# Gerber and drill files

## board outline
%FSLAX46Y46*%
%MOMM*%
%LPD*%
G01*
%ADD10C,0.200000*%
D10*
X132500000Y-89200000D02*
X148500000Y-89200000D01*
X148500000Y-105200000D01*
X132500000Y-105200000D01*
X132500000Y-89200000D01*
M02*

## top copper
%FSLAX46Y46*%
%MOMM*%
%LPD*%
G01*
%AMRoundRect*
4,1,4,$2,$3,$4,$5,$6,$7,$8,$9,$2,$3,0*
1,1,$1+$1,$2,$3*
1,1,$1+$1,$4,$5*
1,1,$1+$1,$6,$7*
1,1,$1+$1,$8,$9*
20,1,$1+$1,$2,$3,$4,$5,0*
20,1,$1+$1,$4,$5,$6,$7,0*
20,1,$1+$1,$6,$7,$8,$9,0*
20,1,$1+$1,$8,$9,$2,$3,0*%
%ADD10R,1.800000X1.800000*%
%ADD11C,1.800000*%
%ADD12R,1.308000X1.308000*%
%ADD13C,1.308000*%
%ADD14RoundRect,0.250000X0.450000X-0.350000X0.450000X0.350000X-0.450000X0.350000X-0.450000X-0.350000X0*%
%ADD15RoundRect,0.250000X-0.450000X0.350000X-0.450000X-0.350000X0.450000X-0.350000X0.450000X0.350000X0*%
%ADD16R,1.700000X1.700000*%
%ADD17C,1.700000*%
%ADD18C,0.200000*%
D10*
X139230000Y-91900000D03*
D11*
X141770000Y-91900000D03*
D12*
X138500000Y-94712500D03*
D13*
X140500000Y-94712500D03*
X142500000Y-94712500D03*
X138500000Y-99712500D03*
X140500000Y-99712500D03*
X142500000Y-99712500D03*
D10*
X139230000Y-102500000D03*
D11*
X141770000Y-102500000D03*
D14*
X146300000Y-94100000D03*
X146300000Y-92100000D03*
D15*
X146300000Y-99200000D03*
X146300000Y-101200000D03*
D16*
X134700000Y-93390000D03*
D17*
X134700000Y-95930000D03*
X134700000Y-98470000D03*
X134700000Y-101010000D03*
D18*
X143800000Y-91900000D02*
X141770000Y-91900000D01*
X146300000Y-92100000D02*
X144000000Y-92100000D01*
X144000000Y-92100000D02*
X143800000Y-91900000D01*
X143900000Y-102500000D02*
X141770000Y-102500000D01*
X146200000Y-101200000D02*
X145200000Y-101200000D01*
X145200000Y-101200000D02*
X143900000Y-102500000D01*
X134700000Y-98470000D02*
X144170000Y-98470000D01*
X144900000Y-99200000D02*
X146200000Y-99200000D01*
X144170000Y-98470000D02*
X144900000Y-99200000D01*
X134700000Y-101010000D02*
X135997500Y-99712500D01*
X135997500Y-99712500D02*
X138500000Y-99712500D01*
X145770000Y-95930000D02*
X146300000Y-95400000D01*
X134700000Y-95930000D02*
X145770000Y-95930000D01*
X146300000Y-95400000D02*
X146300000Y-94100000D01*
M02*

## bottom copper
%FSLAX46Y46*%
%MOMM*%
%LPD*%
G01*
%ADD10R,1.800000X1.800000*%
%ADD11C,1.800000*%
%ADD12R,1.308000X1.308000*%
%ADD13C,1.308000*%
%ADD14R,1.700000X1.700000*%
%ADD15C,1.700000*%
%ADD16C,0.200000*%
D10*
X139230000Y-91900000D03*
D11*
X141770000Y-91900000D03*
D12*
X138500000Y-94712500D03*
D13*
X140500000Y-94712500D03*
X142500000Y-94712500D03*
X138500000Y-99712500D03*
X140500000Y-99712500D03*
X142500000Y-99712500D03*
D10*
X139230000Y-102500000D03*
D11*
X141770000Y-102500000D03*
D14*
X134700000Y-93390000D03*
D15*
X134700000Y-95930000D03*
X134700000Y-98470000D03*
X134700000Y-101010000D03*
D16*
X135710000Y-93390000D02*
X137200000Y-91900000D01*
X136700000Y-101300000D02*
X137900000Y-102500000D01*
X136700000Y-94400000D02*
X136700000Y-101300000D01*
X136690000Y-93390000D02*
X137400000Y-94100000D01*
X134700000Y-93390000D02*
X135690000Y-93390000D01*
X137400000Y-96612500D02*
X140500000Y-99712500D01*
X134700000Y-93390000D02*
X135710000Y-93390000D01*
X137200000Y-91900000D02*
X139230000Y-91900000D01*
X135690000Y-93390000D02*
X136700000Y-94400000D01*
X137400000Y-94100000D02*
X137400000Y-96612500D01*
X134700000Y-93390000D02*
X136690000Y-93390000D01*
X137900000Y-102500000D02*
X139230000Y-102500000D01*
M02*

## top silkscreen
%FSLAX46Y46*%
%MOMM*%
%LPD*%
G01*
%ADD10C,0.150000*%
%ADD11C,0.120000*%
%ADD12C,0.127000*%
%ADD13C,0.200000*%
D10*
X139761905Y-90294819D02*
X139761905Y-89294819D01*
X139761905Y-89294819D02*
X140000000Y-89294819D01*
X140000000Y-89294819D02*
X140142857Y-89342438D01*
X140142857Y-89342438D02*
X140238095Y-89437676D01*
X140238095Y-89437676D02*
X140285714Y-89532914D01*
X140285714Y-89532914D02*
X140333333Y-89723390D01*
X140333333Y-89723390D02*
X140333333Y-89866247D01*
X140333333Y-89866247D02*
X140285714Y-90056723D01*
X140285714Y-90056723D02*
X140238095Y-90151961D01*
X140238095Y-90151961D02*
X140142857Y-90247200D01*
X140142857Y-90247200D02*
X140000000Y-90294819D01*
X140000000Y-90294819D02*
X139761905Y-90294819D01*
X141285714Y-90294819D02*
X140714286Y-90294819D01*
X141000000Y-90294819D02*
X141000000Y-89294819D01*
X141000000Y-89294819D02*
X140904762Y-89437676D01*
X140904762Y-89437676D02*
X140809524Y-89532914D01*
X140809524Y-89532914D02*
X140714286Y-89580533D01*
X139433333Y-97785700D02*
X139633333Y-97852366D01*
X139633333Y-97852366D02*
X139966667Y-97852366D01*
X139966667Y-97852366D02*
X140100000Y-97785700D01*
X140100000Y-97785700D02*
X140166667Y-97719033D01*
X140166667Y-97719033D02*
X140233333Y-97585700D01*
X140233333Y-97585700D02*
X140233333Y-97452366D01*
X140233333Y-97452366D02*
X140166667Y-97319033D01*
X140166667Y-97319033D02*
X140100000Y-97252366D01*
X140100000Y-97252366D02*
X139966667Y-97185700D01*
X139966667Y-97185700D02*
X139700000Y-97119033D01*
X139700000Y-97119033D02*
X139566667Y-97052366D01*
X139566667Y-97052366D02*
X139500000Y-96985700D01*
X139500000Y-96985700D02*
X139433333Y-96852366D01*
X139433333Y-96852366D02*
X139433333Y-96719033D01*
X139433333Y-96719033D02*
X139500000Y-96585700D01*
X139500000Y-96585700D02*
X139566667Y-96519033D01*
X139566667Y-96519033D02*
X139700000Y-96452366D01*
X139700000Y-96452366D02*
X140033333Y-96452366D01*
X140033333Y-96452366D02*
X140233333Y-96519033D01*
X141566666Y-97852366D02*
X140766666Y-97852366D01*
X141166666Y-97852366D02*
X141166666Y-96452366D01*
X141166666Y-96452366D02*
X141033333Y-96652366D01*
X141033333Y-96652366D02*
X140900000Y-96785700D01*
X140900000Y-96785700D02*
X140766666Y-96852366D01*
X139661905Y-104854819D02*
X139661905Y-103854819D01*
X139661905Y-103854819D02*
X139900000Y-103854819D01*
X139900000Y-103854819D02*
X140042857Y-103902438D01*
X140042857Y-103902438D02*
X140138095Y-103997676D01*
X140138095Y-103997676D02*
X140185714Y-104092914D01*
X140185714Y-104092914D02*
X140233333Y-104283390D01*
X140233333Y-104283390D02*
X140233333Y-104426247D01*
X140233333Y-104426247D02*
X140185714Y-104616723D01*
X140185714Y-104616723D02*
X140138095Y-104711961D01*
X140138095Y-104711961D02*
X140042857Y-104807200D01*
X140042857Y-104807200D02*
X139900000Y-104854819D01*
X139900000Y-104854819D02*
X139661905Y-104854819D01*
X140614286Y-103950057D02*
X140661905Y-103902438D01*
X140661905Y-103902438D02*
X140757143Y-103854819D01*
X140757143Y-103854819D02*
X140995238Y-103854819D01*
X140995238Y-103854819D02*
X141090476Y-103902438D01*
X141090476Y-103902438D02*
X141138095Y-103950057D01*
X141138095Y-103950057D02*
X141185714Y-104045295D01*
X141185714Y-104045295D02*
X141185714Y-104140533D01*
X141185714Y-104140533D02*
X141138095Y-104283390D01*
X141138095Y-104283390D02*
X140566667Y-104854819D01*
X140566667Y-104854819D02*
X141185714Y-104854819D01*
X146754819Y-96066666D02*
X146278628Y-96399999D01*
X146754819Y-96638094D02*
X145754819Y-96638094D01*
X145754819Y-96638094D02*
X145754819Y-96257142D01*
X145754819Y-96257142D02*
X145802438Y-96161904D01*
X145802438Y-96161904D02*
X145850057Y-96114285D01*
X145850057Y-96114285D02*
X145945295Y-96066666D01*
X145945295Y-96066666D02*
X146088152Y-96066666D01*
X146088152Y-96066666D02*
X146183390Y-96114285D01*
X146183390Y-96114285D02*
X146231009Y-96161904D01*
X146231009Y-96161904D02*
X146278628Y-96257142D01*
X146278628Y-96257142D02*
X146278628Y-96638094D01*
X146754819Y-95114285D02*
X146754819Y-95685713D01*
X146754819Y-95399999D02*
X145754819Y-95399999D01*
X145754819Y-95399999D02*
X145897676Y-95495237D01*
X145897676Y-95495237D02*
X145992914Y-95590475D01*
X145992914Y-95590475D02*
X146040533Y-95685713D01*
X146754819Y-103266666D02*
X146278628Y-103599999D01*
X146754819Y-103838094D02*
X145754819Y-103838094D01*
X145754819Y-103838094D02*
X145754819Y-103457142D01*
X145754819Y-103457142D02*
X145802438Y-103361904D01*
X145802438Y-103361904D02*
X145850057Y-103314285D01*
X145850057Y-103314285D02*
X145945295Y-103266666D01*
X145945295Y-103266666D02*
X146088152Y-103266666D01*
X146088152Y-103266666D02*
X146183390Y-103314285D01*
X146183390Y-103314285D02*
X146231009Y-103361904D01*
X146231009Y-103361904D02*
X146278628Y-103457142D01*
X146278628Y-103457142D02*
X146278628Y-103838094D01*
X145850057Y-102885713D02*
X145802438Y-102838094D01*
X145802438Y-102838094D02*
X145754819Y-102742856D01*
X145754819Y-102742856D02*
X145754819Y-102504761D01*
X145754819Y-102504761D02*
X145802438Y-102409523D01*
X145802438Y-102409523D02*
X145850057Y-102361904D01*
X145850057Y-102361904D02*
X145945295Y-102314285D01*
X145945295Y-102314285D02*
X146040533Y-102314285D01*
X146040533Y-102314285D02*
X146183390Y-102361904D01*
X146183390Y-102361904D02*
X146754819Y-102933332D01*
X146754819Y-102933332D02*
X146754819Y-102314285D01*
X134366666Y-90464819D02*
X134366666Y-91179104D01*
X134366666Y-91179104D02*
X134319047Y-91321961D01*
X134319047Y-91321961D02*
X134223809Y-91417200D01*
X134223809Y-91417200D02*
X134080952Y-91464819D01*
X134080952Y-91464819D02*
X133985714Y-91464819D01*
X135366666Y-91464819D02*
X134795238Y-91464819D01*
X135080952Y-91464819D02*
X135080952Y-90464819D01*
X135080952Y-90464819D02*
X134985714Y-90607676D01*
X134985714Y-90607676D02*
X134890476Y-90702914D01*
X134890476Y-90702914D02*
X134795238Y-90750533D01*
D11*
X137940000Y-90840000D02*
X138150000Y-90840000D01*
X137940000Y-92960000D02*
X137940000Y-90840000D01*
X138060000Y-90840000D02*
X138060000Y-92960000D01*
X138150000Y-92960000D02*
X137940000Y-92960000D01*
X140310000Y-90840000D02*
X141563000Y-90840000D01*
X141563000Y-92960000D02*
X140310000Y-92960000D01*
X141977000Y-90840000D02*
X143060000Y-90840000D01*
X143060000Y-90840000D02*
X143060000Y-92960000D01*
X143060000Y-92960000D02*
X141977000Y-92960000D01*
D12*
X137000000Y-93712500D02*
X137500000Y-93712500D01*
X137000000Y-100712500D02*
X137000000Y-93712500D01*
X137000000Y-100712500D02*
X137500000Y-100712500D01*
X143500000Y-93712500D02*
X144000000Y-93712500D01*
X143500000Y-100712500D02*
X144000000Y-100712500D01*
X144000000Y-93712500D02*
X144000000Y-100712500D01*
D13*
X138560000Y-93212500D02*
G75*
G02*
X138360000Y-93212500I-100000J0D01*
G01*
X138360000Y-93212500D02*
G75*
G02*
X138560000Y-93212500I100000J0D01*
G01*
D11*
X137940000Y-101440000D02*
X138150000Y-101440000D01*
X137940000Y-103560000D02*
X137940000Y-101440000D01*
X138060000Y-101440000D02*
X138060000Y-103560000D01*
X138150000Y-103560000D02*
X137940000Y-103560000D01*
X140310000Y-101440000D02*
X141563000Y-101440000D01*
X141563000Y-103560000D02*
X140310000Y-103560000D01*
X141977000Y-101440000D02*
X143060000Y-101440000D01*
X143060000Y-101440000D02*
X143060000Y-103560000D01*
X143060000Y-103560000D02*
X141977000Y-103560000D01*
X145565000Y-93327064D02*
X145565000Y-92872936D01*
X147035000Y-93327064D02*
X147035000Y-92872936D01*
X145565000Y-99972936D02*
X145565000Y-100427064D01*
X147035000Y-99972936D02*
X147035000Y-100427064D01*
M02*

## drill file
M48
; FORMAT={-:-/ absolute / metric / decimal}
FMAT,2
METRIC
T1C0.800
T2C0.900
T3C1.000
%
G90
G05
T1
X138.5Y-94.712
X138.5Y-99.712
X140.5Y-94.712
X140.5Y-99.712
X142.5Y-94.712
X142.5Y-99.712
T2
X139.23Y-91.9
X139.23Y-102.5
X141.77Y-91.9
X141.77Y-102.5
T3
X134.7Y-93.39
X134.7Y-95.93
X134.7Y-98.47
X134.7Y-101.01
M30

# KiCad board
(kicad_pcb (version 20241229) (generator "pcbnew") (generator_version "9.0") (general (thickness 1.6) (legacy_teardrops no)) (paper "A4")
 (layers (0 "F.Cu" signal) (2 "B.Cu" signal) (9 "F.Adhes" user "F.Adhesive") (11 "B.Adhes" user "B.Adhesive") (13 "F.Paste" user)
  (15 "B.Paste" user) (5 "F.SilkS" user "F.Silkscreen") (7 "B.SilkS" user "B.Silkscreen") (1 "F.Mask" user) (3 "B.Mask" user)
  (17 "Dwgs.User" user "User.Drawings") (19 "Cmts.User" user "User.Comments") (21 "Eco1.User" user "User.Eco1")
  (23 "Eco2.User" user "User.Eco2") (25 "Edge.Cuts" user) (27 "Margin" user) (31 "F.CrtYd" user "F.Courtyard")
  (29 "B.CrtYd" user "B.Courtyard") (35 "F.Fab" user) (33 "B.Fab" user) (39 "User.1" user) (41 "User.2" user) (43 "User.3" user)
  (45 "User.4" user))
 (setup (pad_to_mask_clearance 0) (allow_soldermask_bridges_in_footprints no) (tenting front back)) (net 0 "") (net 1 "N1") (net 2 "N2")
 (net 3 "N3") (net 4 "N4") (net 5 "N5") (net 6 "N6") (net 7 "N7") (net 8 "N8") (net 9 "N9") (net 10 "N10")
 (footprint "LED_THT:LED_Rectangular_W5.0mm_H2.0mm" (layer "F.Cu") (at 139.23 91.9)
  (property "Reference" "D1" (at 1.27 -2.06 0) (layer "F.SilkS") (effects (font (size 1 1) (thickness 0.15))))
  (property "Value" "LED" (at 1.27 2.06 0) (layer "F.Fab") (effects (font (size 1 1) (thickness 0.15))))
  (fp_line (start -1.29 -1.06) (end -1.08 -1.06) (stroke (width 0.12) (type solid)) (layer "F.SilkS"))
  (fp_line (start -1.29 1.06) (end -1.29 -1.06) (stroke (width 0.12) (type solid)) (layer "F.SilkS"))
  (fp_line (start -1.17 -1.06) (end -1.17 1.06) (stroke (width 0.12) (type solid)) (layer "F.SilkS"))
  (fp_line (start -1.08 1.06) (end -1.29 1.06) (stroke (width 0.12) (type solid)) (layer "F.SilkS"))
  (fp_line (start 1.08 -1.06) (end 2.333 -1.06) (stroke (width 0.12) (type solid)) (layer "F.SilkS"))
  (fp_line (start 2.333 1.06) (end 1.08 1.06) (stroke (width 0.12) (type solid)) (layer "F.SilkS"))
  (fp_line (start 2.747 -1.06) (end 3.83 -1.06) (stroke (width 0.12) (type solid)) (layer "F.SilkS"))
  (fp_line (start 3.83 -1.06) (end 3.83 1.06) (stroke (width 0.12) (type solid)) (layer "F.SilkS"))
  (fp_line (start 3.83 1.06) (end 2.747 1.06) (stroke (width 0.12) (type solid)) (layer "F.SilkS"))
  (pad "1" thru_hole rect (at 0 0) (size 1.8 1.8) (drill 0.9) (layers "*.Cu" "*.Mask") (remove_unused_layers no) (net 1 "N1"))
  (pad "2" thru_hole circle (at 2.54 0) (size 1.8 1.8) (drill 0.9) (layers "*.Cu" "*.Mask") (remove_unused_layers no) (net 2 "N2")))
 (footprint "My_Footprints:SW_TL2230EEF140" (layer "F.Cu") (at 140.5 97.2125)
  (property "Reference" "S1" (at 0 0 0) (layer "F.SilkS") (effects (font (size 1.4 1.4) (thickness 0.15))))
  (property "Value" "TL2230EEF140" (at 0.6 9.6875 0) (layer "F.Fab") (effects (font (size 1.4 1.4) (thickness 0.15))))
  (fp_line (start -3.5 -3.5) (end -3 -3.5) (stroke (width 0.127) (type solid)) (layer "F.SilkS"))
  (fp_line (start -3.5 3.5) (end -3.5 -3.5) (stroke (width 0.127) (type solid)) (layer "F.SilkS"))
  (fp_line (start -3.5 3.5) (end -3 3.5) (stroke (width 0.127) (type solid)) (layer "F.SilkS"))
  (fp_line (start 3 -3.5) (end 3.5 -3.5) (stroke (width 0.127) (type solid)) (layer "F.SilkS"))
  (fp_line (start 3 3.5) (end 3.5 3.5) (stroke (width 0.127) (type solid)) (layer "F.SilkS"))
  (fp_line (start 3.5 -3.5) (end 3.5 3.5) (stroke (width 0.127) (type solid)) (layer "F.SilkS"))
  (fp_circle (center -2.04 -4) (end -1.94 -4) (stroke (width 0.2) (type solid)) (fill no) (layer "F.SilkS"))
  (pad "1" thru_hole rect (at -2 -2.5) (size 1.308 1.308) (drill 0.8) (layers "*.Cu" "*.Mask") (remove_unused_layers no) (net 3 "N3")
   (solder_mask_margin 0.102))
  (pad "2" thru_hole circle (at 0 -2.5) (size 1.308 1.308) (drill 0.8) (layers "*.Cu" "*.Mask") (remove_unused_layers no) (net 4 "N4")
   (solder_mask_margin 0.102))
  (pad "3" thru_hole circle (at 2 -2.5) (size 1.308 1.308) (drill 0.8) (layers "*.Cu" "*.Mask") (remove_unused_layers no) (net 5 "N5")
   (solder_mask_margin 0.102))
  (pad "4" thru_hole circle (at -2 2.5) (size 1.308 1.308) (drill 0.8) (layers "*.Cu" "*.Mask") (remove_unused_layers no) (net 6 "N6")
   (solder_mask_margin 0.102))
  (pad "5" thru_hole circle (at 0 2.5) (size 1.308 1.308) (drill 0.8) (layers "*.Cu" "*.Mask") (remove_unused_layers no) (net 1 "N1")
   (solder_mask_margin 0.102))
  (pad "6" thru_hole circle (at 2 2.5) (size 1.308 1.308) (drill 0.8) (layers "*.Cu" "*.Mask") (remove_unused_layers no) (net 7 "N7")
   (solder_mask_margin 0.102)))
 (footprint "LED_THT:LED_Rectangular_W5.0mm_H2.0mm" (layer "F.Cu") (at 139.23 102.5)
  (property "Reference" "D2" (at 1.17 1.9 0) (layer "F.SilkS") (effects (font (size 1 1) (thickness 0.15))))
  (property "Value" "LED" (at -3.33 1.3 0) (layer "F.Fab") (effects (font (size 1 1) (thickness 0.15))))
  (fp_line (start -1.29 -1.06) (end -1.08 -1.06) (stroke (width 0.12) (type solid)) (layer "F.SilkS"))
  (fp_line (start -1.29 1.06) (end -1.29 -1.06) (stroke (width 0.12) (type solid)) (layer "F.SilkS"))
  (fp_line (start -1.17 -1.06) (end -1.17 1.06) (stroke (width 0.12) (type solid)) (layer "F.SilkS"))
  (fp_line (start -1.08 1.06) (end -1.29 1.06) (stroke (width 0.12) (type solid)) (layer "F.SilkS"))
  (fp_line (start 1.08 -1.06) (end 2.333 -1.06) (stroke (width 0.12) (type solid)) (layer "F.SilkS"))
  (fp_line (start 2.333 1.06) (end 1.08 1.06) (stroke (width 0.12) (type solid)) (layer "F.SilkS"))
  (fp_line (start 2.747 -1.06) (end 3.83 -1.06) (stroke (width 0.12) (type solid)) (layer "F.SilkS"))
  (fp_line (start 3.83 -1.06) (end 3.83 1.06) (stroke (width 0.12) (type solid)) (layer "F.SilkS"))
  (fp_line (start 3.83 1.06) (end 2.747 1.06) (stroke (width 0.12) (type solid)) (layer "F.SilkS"))
  (pad "1" thru_hole rect (at 0 0) (size 1.8 1.8) (drill 0.9) (layers "*.Cu" "*.Mask") (remove_unused_layers no) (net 1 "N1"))
  (pad "2" thru_hole circle (at 2.54 0) (size 1.8 1.8) (drill 0.9) (layers "*.Cu" "*.Mask") (remove_unused_layers no) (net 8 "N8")))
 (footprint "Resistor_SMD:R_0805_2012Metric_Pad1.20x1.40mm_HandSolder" (layer "F.Cu") (at 146.3 93.1 90)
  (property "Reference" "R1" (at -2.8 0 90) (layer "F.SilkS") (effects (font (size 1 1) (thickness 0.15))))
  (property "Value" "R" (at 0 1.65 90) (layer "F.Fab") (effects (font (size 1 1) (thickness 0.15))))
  (fp_line (start -0.227064 -0.735) (end 0.227064 -0.735) (stroke (width 0.12) (type solid)) (layer "F.SilkS"))
  (fp_line (start -0.227064 0.735) (end 0.227064 0.735) (stroke (width 0.12) (type solid)) (layer "F.SilkS"))
  (pad "1" smd roundrect (at -1 0 90) (size 1.2 1.4) (layers "F.Cu" "F.Mask" "F.Paste") (roundrect_rratio 0.208333) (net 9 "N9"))
  (pad "2" smd roundrect (at 1 0 90) (size 1.2 1.4) (layers "F.Cu" "F.Mask" "F.Paste") (roundrect_rratio 0.208333) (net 2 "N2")))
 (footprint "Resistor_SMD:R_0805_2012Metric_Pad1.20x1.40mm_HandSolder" (layer "F.Cu") (at 146.3 100.2 -90)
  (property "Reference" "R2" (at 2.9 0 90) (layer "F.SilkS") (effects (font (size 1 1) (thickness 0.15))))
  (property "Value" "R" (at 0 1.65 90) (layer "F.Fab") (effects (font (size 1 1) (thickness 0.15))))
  (fp_line (start -0.227064 0.735) (end 0.227064 0.735) (stroke (width 0.12) (type solid)) (layer "F.SilkS"))
  (fp_line (start -0.227064 -0.735) (end 0.227064 -0.735) (stroke (width 0.12) (type solid)) (layer "F.SilkS"))
  (pad "1" smd roundrect (at -1 0 270) (size 1.2 1.4) (layers "F.Cu" "F.Mask" "F.Paste") (roundrect_rratio 0.208333) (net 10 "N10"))
  (pad "2" smd roundrect (at 1 0 270) (size 1.2 1.4) (layers "F.Cu" "F.Mask" "F.Paste") (roundrect_rratio 0.208333) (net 8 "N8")))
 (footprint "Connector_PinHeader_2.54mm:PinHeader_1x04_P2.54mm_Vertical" (layer "B.Cu") (at 134.7 93.39 180)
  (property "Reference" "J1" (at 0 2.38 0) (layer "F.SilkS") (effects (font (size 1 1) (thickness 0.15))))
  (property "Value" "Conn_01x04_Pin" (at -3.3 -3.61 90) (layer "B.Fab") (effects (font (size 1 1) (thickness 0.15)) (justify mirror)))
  (pad "1" thru_hole rect (at 0 0 180) (size 1.7 1.7) (drill 1) (layers "*.Cu" "*.Mask") (remove_unused_layers no) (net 1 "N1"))
  (pad "2" thru_hole circle (at 0 -2.54 180) (size 1.7 1.7) (drill 1) (layers "*.Cu" "*.Mask") (remove_unused_layers no) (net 9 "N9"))
  (pad "3" thru_hole circle (at 0 -5.08 180) (size 1.7 1.7) (drill 1) (layers "*.Cu" "*.Mask") (remove_unused_layers no) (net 10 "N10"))
  (pad "4" thru_hole circle (at 0 -7.62 180) (size 1.7 1.7) (drill 1) (layers "*.Cu" "*.Mask") (remove_unused_layers no) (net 6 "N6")))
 (gr_rect (start 132.5 89.2) (end 148.5 105.2) (stroke (width 0.2) (type solid)) (fill no) (layer "Edge.Cuts"))
 (segment (start 135.71 93.39) (end 137.2 91.9) (width 0.2) (layer "B.Cu") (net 1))
 (segment (start 136.7 101.3) (end 137.9 102.5) (width 0.2) (layer "B.Cu") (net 1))
 (segment (start 136.7 94.4) (end 136.7 101.3) (width 0.2) (layer "B.Cu") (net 1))
 (segment (start 136.69 93.39) (end 137.4 94.1) (width 0.2) (layer "B.Cu") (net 1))
 (segment (start 134.7 93.39) (end 135.69 93.39) (width 0.2) (layer "B.Cu") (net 1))
 (segment (start 137.4 96.6125) (end 140.5 99.7125) (width 0.2) (layer "B.Cu") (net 1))
 (segment (start 134.7 93.39) (end 135.71 93.39) (width 0.2) (layer "B.Cu") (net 1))
 (segment (start 137.2 91.9) (end 139.23 91.9) (width 0.2) (layer "B.Cu") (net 1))
 (segment (start 135.69 93.39) (end 136.7 94.4) (width 0.2) (layer "B.Cu") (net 1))
 (segment (start 137.4 94.1) (end 137.4 96.6125) (width 0.2) (layer "B.Cu") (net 1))
 (segment (start 134.7 93.39) (end 136.69 93.39) (width 0.2) (layer "B.Cu") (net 1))
 (segment (start 137.9 102.5) (end 139.23 102.5) (width 0.2) (layer "B.Cu") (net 1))
 (segment (start 143.8 91.9) (end 141.77 91.9) (width 0.2) (layer "F.Cu") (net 2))
 (segment (start 146.3 92.1) (end 144 92.1) (width 0.2) (layer "F.Cu") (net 2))
 (segment (start 144 92.1) (end 143.8 91.9) (width 0.2) (layer "F.Cu") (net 2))
 (segment (start 143.9 102.5) (end 141.77 102.5) (width 0.2) (layer "F.Cu") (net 8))
 (segment (start 146.2 101.2) (end 145.2 101.2) (width 0.2) (layer "F.Cu") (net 8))
 (segment (start 145.2 101.2) (end 143.9 102.5) (width 0.2) (layer "F.Cu") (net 8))
 (segment (start 134.7 98.47) (end 144.17 98.47) (width 0.2) (layer "F.Cu") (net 10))
 (segment (start 144.9 99.2) (end 146.2 99.2) (width 0.2) (layer "F.Cu") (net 10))
 (segment (start 144.17 98.47) (end 144.9 99.2) (width 0.2) (layer "F.Cu") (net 10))
 (segment (start 134.7 101.01) (end 135.9975 99.7125) (width 0.2) (layer "F.Cu") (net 6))
 (segment (start 135.9975 99.7125) (end 138.5 99.7125) (width 0.2) (layer "F.Cu") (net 6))
 (segment (start 145.77 95.93) (end 146.3 95.4) (width 0.2) (layer "F.Cu") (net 9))
 (segment (start 134.7 95.93) (end 145.77 95.93) (width 0.2) (layer "F.Cu") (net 9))
 (segment (start 146.3 95.4) (end 146.3 94.1) (width 0.2) (layer "F.Cu") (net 9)))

